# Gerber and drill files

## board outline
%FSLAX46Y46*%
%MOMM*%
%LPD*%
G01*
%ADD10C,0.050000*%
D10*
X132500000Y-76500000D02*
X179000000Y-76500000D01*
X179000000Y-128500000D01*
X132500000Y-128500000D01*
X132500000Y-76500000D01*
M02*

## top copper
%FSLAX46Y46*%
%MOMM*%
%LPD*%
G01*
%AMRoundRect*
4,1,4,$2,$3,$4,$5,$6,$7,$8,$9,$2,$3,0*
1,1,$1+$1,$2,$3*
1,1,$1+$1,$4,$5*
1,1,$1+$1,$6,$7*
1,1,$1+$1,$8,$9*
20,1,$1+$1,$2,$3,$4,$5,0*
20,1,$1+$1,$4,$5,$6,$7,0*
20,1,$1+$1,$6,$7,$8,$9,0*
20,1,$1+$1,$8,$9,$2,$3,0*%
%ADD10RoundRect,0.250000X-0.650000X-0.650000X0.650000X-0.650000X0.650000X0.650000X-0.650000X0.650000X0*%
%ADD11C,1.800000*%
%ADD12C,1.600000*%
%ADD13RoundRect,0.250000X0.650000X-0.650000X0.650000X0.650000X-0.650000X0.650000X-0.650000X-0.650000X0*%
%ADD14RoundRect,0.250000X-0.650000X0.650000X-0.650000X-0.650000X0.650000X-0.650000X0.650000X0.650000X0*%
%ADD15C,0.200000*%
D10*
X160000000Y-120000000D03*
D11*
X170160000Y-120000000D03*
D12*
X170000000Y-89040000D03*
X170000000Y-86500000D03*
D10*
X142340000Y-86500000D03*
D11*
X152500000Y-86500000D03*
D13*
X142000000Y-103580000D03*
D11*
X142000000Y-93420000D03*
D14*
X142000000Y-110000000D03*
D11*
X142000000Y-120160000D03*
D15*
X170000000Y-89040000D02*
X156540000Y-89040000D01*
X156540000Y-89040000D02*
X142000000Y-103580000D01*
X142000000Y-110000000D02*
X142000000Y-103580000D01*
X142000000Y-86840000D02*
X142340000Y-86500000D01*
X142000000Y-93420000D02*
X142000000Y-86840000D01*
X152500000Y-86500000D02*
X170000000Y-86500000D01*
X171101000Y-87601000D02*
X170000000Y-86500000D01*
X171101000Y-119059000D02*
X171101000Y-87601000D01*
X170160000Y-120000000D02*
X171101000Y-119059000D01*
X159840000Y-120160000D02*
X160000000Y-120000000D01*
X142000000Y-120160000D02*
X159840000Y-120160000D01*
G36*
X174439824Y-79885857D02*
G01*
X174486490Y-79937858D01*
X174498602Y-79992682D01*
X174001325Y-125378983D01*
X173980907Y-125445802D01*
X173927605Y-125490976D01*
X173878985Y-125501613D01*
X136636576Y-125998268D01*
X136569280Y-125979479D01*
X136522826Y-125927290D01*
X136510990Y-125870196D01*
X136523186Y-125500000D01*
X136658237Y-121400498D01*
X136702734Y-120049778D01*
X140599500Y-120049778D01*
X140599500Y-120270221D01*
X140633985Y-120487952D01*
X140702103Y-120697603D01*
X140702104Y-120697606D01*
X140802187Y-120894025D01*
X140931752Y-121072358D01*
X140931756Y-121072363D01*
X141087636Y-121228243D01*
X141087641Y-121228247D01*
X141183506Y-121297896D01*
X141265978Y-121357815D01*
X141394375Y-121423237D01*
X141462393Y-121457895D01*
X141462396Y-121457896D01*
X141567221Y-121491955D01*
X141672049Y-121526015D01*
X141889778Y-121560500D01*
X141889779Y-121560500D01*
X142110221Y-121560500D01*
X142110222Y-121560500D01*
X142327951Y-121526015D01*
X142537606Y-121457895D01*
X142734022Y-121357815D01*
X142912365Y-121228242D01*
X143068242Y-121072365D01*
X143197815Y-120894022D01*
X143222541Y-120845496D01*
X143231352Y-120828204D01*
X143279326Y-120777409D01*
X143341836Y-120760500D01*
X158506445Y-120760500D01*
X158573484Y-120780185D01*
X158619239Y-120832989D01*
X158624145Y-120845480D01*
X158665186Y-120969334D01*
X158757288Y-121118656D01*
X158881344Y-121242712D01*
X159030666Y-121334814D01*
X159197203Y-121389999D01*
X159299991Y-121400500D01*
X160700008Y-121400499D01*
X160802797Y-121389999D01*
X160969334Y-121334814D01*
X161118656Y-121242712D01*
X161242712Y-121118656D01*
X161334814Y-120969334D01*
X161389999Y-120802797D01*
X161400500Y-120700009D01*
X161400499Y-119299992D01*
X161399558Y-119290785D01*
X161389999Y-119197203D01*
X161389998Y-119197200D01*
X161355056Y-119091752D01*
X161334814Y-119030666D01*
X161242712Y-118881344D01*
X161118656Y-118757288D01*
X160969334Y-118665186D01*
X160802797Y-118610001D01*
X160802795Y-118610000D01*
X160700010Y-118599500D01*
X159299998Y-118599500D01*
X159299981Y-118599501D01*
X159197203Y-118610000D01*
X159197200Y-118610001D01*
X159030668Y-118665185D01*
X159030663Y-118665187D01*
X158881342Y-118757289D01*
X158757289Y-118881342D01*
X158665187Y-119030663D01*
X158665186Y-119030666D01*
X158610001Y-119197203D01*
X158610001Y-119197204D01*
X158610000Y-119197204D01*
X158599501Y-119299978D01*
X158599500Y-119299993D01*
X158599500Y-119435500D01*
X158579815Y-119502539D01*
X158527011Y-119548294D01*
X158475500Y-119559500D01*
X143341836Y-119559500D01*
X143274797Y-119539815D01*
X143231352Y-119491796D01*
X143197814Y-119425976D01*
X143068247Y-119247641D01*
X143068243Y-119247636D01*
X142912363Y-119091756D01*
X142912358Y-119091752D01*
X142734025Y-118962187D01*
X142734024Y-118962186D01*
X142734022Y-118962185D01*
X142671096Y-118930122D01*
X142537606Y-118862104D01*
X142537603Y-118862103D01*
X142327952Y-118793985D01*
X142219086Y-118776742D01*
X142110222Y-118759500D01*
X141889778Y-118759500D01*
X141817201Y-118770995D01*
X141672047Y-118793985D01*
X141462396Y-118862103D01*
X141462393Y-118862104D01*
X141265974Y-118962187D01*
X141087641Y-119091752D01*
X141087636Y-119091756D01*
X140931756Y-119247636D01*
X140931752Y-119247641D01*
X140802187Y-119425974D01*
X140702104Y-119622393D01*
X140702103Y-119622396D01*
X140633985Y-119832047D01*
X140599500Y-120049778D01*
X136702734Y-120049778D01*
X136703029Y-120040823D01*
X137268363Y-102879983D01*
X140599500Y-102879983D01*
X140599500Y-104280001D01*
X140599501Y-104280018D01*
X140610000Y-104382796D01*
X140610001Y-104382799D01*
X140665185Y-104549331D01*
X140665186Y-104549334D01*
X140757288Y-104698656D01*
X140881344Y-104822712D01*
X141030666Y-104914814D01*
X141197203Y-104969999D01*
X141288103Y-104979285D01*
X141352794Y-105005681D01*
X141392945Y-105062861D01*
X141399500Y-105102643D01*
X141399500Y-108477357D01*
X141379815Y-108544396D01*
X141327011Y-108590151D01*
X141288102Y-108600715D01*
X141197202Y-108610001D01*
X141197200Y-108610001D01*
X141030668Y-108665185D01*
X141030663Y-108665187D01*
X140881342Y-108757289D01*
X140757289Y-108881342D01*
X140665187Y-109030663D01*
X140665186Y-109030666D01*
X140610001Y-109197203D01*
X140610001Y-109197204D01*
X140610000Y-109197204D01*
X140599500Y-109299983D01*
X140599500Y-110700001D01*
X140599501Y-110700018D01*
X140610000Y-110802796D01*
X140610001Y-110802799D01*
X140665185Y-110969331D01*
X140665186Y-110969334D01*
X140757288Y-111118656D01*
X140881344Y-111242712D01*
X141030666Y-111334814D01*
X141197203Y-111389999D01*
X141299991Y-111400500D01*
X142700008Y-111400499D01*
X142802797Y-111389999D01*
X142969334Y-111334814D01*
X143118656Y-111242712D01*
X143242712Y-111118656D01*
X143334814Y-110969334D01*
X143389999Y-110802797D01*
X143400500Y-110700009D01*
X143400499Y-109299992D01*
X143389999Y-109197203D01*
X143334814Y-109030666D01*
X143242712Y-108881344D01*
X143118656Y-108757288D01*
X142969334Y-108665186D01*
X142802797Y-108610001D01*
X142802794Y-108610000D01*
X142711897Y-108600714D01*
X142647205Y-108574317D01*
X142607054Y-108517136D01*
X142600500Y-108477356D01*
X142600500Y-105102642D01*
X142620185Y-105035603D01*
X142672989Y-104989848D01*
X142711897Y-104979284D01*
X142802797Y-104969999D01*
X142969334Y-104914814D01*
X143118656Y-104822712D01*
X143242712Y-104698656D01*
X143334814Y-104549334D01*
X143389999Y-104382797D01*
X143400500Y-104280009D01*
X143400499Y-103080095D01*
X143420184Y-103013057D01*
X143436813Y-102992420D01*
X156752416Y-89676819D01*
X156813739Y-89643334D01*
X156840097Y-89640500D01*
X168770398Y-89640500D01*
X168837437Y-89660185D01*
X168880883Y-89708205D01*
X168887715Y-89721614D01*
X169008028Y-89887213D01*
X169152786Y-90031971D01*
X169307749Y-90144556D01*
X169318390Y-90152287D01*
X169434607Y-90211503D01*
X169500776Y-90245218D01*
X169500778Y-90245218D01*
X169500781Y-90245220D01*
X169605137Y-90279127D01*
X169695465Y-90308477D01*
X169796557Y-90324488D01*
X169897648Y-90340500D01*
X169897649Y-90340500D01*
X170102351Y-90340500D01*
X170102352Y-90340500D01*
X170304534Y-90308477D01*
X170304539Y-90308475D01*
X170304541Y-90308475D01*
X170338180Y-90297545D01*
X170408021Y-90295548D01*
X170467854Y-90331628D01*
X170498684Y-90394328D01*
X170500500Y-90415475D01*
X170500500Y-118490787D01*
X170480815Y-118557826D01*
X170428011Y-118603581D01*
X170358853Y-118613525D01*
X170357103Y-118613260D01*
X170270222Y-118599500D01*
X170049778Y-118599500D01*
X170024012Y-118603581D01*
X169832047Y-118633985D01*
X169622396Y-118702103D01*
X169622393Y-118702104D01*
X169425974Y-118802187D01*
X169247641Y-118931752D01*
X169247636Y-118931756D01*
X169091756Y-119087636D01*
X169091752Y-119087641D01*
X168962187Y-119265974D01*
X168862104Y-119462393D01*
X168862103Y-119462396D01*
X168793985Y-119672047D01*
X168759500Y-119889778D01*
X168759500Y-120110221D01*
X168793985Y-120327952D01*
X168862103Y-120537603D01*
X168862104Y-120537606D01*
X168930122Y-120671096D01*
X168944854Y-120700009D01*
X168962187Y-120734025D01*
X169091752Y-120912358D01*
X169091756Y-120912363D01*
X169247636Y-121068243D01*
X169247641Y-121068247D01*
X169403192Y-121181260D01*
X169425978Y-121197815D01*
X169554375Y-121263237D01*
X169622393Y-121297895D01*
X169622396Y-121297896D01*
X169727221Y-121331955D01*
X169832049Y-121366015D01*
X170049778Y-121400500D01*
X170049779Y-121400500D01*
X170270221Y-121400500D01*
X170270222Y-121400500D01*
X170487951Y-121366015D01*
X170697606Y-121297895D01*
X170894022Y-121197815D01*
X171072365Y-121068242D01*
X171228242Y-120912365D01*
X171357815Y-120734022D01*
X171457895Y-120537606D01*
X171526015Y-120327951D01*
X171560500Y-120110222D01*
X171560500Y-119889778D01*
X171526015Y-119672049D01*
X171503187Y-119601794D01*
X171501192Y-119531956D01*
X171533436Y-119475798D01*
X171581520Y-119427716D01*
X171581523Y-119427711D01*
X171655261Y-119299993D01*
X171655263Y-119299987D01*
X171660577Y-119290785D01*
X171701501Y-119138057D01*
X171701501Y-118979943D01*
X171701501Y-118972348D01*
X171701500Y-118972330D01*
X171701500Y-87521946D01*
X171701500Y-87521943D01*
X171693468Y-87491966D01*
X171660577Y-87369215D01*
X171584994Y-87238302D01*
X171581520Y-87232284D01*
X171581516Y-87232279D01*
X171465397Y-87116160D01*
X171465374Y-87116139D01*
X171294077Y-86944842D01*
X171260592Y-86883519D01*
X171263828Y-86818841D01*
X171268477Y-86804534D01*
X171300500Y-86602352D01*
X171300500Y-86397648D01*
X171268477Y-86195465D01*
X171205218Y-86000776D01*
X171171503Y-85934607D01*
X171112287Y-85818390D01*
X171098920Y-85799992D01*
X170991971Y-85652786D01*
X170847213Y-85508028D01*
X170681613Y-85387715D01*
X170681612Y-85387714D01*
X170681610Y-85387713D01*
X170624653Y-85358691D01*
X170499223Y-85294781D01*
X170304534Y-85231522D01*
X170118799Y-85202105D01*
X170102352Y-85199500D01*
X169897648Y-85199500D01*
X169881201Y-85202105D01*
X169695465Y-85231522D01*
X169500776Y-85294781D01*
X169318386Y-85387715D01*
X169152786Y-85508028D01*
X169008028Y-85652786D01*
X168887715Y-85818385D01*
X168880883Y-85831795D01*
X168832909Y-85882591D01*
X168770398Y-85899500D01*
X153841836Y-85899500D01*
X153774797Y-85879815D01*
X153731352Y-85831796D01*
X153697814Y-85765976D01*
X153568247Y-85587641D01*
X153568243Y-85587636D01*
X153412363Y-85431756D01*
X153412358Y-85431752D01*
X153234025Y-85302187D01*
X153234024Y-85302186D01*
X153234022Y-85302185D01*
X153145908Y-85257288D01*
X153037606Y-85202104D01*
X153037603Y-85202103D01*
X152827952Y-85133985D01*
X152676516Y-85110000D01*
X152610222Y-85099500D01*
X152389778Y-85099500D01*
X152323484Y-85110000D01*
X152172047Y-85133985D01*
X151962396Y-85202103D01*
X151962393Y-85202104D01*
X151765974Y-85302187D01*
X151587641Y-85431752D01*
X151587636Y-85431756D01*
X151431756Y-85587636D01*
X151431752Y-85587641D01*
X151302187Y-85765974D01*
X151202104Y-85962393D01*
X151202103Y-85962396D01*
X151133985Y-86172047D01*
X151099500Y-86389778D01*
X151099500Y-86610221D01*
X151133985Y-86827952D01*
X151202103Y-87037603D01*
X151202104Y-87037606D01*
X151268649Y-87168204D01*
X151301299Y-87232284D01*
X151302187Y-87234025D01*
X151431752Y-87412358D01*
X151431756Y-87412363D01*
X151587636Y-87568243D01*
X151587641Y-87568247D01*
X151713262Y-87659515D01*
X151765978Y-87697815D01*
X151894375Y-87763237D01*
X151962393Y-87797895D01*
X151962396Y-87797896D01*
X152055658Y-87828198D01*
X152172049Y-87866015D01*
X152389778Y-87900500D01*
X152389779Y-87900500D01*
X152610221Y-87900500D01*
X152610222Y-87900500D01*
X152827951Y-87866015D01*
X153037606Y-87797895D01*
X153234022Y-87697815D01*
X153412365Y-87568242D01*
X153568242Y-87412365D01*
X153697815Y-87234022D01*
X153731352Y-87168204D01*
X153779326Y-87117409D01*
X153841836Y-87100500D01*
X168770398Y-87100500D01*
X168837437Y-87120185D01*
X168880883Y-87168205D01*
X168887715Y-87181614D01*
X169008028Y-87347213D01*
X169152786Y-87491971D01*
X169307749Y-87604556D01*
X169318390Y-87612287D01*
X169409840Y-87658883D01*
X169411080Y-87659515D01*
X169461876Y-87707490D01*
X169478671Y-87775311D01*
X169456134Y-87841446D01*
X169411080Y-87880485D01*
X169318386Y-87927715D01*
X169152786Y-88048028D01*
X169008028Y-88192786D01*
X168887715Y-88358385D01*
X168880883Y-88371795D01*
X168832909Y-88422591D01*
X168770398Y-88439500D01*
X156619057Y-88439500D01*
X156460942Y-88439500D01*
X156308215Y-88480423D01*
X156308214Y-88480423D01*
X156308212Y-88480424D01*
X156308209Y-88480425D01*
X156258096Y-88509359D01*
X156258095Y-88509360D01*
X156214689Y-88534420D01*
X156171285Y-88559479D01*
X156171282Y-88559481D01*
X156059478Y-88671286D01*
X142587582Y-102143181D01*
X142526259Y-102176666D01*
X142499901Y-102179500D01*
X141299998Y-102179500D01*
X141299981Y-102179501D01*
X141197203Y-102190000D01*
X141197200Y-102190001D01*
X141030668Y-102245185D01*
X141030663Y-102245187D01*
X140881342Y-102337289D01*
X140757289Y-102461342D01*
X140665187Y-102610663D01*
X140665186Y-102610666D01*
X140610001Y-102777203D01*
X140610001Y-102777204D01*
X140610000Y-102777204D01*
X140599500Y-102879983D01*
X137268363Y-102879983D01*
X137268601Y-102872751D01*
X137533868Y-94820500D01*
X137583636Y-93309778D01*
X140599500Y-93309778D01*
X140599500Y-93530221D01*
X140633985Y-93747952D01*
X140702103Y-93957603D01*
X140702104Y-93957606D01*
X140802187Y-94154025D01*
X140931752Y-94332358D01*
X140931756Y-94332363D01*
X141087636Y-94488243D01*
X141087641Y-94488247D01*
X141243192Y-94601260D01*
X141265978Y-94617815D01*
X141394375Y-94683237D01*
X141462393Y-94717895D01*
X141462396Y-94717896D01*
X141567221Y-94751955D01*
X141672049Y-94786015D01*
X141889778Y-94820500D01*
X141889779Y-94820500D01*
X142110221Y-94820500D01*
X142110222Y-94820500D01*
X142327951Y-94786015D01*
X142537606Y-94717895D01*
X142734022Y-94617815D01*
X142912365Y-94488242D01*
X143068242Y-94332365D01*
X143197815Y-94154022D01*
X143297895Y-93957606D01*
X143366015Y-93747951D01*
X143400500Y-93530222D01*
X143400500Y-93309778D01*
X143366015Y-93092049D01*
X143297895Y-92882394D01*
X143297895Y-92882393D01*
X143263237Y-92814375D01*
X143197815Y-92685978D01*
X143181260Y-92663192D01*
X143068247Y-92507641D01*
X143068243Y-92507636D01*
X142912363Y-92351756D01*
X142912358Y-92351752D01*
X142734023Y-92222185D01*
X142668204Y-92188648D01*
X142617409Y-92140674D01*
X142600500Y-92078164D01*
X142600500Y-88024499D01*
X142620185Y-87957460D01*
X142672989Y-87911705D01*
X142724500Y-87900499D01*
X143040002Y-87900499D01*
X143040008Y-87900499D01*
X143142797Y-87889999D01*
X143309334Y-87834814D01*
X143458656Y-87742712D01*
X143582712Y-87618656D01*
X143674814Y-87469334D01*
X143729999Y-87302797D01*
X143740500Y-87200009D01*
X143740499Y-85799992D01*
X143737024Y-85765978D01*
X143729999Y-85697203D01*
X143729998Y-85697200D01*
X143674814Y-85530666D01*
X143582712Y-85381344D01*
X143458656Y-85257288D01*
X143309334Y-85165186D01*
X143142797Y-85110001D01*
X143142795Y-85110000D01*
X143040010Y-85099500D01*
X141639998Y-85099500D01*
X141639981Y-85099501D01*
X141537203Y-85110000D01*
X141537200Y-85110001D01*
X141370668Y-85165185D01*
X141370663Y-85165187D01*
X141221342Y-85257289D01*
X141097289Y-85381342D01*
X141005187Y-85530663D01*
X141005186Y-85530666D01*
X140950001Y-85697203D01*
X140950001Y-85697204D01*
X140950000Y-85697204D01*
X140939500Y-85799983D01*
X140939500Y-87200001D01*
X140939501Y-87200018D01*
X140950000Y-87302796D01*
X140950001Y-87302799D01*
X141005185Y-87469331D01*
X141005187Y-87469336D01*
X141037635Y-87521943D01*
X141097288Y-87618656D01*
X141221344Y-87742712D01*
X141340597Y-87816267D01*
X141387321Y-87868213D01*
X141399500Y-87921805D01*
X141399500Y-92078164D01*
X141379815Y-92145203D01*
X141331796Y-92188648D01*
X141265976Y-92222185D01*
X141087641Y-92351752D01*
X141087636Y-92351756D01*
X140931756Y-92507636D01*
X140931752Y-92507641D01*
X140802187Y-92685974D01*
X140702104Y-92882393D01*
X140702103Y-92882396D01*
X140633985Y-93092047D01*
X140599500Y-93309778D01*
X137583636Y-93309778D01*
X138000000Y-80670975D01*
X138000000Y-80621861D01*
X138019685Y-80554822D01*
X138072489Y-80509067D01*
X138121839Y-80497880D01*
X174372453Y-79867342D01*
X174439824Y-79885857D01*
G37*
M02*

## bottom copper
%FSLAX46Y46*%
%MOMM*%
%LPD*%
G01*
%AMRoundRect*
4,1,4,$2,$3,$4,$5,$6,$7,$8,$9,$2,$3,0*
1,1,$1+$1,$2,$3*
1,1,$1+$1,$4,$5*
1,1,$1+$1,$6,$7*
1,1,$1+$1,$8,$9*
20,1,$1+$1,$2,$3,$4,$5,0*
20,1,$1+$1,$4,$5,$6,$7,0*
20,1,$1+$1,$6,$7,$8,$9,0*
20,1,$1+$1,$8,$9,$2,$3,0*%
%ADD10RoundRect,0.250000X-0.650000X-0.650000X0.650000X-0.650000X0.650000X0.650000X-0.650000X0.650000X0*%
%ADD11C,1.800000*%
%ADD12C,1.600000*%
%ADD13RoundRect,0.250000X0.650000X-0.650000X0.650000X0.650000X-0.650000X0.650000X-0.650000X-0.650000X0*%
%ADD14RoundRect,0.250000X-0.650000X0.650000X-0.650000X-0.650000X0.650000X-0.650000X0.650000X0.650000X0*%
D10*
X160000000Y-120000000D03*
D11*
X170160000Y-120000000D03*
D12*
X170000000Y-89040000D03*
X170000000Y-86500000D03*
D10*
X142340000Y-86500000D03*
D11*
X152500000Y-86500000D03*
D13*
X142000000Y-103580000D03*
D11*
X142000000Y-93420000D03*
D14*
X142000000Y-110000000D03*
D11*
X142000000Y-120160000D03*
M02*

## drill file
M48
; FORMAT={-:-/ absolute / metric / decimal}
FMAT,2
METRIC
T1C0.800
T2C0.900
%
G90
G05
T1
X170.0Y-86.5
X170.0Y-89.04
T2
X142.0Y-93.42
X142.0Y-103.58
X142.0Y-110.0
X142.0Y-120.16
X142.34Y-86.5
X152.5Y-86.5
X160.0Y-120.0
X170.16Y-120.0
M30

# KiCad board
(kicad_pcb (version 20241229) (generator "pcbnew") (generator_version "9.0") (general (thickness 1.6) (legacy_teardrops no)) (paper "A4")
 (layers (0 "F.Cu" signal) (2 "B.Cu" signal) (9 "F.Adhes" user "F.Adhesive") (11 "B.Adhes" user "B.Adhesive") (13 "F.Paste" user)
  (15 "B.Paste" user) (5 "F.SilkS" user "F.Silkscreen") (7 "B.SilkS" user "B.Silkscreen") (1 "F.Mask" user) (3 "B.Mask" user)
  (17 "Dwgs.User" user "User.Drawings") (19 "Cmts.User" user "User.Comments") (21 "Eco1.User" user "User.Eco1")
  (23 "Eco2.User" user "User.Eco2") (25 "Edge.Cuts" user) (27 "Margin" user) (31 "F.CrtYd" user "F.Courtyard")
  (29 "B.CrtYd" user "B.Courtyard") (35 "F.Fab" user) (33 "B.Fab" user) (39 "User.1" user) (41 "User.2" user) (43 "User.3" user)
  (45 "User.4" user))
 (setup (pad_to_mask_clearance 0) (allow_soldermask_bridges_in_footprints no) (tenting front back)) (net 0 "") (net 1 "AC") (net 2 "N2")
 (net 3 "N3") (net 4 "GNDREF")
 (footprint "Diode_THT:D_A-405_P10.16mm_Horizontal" (layer "F.Cu") (at 160 120)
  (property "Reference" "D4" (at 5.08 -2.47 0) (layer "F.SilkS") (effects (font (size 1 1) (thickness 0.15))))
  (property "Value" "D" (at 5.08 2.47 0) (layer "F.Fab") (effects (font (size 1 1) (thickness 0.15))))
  (pad "1" thru_hole roundrect (at 0 0) (size 1.8 1.8) (drill 0.9) (layers "*.Cu" "*.Mask") (remove_unused_layers no)
   (roundrect_rratio 0.138889) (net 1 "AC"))
  (pad "2" thru_hole circle (at 10.16 0) (size 1.8 1.8) (drill 0.9) (layers "*.Cu" "*.Mask") (remove_unused_layers no) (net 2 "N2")))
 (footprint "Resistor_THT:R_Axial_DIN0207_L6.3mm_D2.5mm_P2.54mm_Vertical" (layer "F.Cu") (at 170 89.04 90)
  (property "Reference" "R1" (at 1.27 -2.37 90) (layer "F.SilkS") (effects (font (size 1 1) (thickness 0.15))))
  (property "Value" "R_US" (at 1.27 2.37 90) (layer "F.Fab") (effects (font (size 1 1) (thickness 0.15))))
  (pad "1" thru_hole circle (at 0 0 90) (size 1.6 1.6) (drill 0.8) (layers "*.Cu" "*.Mask") (remove_unused_layers no) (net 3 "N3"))
  (pad "2" thru_hole circle (at 2.54 0 90) (size 1.6 1.6) (drill 0.8) (layers "*.Cu" "*.Mask") (remove_unused_layers no) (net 2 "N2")))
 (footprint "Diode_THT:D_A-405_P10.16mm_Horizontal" (layer "F.Cu") (at 142.34 86.5)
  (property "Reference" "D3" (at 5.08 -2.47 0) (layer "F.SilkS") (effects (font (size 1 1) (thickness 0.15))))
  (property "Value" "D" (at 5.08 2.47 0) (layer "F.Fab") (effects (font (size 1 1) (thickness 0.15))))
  (pad "1" thru_hole roundrect (at 0 0) (size 1.8 1.8) (drill 0.9) (layers "*.Cu" "*.Mask") (remove_unused_layers no)
   (roundrect_rratio 0.138889) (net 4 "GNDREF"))
  (pad "2" thru_hole circle (at 10.16 0) (size 1.8 1.8) (drill 0.9) (layers "*.Cu" "*.Mask") (remove_unused_layers no) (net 2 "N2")))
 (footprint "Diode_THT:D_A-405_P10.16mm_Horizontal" (layer "F.Cu") (at 142 103.58 90)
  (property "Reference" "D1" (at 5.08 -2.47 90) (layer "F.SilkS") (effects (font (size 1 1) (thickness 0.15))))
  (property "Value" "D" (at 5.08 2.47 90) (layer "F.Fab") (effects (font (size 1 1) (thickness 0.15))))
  (pad "1" thru_hole roundrect (at 0 0 90) (size 1.8 1.8) (drill 0.9) (layers "*.Cu" "*.Mask") (remove_unused_layers no)
   (roundrect_rratio 0.138889) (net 3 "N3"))
  (pad "2" thru_hole circle (at 10.16 0 90) (size 1.8 1.8) (drill 0.9) (layers "*.Cu" "*.Mask") (remove_unused_layers no) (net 4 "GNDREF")))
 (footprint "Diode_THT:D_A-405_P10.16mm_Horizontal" (layer "F.Cu") (at 142 110 -90)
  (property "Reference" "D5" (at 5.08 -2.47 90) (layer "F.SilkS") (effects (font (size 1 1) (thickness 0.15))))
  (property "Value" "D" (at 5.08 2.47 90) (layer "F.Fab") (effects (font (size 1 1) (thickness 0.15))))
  (pad "1" thru_hole roundrect (at 0 0 270) (size 1.8 1.8) (drill 0.9) (layers "*.Cu" "*.Mask") (remove_unused_layers no)
   (roundrect_rratio 0.138889) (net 3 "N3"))
  (pad "2" thru_hole circle (at 10.16 0 270) (size 1.8 1.8) (drill 0.9) (layers "*.Cu" "*.Mask") (remove_unused_layers no) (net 1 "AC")))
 (gr_rect (start 132.5 76.5) (end 179 128.5) (stroke (width 0.05) (type default)) (fill no) (layer "Edge.Cuts"))
 (segment (start 170 89.04) (end 156.54 89.04) (width 0.2) (layer "F.Cu") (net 3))
 (segment (start 156.54 89.04) (end 142 103.58) (width 0.2) (layer "F.Cu") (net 3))
 (segment (start 142 110) (end 142 103.58) (width 0.2) (layer "F.Cu") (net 3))
 (segment (start 142 86.84) (end 142.34 86.5) (width 0.2) (layer "F.Cu") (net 4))
 (segment (start 142 93.42) (end 142 86.84) (width 0.2) (layer "F.Cu") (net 4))
 (segment (start 152.5 86.5) (end 170 86.5) (width 0.2) (layer "F.Cu") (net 2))
 (segment (start 171.101 87.601) (end 170 86.5) (width 0.2) (layer "F.Cu") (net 2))
 (segment (start 171.101 119.059) (end 171.101 87.601) (width 0.2) (layer "F.Cu") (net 2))
 (segment (start 170.16 120) (end 171.101 119.059) (width 0.2) (layer "F.Cu") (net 2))
 (segment (start 159.84 120.16) (end 160 120) (width 0.2) (layer "F.Cu") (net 1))
 (segment (start 142 120.16) (end 159.84 120.16) (width 0.2) (layer "F.Cu") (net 1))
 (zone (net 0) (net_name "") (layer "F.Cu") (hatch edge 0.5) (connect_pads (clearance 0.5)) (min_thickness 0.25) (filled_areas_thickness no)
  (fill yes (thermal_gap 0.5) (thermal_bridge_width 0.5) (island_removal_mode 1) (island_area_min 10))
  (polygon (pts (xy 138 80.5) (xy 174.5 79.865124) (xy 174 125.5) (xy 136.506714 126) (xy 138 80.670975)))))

